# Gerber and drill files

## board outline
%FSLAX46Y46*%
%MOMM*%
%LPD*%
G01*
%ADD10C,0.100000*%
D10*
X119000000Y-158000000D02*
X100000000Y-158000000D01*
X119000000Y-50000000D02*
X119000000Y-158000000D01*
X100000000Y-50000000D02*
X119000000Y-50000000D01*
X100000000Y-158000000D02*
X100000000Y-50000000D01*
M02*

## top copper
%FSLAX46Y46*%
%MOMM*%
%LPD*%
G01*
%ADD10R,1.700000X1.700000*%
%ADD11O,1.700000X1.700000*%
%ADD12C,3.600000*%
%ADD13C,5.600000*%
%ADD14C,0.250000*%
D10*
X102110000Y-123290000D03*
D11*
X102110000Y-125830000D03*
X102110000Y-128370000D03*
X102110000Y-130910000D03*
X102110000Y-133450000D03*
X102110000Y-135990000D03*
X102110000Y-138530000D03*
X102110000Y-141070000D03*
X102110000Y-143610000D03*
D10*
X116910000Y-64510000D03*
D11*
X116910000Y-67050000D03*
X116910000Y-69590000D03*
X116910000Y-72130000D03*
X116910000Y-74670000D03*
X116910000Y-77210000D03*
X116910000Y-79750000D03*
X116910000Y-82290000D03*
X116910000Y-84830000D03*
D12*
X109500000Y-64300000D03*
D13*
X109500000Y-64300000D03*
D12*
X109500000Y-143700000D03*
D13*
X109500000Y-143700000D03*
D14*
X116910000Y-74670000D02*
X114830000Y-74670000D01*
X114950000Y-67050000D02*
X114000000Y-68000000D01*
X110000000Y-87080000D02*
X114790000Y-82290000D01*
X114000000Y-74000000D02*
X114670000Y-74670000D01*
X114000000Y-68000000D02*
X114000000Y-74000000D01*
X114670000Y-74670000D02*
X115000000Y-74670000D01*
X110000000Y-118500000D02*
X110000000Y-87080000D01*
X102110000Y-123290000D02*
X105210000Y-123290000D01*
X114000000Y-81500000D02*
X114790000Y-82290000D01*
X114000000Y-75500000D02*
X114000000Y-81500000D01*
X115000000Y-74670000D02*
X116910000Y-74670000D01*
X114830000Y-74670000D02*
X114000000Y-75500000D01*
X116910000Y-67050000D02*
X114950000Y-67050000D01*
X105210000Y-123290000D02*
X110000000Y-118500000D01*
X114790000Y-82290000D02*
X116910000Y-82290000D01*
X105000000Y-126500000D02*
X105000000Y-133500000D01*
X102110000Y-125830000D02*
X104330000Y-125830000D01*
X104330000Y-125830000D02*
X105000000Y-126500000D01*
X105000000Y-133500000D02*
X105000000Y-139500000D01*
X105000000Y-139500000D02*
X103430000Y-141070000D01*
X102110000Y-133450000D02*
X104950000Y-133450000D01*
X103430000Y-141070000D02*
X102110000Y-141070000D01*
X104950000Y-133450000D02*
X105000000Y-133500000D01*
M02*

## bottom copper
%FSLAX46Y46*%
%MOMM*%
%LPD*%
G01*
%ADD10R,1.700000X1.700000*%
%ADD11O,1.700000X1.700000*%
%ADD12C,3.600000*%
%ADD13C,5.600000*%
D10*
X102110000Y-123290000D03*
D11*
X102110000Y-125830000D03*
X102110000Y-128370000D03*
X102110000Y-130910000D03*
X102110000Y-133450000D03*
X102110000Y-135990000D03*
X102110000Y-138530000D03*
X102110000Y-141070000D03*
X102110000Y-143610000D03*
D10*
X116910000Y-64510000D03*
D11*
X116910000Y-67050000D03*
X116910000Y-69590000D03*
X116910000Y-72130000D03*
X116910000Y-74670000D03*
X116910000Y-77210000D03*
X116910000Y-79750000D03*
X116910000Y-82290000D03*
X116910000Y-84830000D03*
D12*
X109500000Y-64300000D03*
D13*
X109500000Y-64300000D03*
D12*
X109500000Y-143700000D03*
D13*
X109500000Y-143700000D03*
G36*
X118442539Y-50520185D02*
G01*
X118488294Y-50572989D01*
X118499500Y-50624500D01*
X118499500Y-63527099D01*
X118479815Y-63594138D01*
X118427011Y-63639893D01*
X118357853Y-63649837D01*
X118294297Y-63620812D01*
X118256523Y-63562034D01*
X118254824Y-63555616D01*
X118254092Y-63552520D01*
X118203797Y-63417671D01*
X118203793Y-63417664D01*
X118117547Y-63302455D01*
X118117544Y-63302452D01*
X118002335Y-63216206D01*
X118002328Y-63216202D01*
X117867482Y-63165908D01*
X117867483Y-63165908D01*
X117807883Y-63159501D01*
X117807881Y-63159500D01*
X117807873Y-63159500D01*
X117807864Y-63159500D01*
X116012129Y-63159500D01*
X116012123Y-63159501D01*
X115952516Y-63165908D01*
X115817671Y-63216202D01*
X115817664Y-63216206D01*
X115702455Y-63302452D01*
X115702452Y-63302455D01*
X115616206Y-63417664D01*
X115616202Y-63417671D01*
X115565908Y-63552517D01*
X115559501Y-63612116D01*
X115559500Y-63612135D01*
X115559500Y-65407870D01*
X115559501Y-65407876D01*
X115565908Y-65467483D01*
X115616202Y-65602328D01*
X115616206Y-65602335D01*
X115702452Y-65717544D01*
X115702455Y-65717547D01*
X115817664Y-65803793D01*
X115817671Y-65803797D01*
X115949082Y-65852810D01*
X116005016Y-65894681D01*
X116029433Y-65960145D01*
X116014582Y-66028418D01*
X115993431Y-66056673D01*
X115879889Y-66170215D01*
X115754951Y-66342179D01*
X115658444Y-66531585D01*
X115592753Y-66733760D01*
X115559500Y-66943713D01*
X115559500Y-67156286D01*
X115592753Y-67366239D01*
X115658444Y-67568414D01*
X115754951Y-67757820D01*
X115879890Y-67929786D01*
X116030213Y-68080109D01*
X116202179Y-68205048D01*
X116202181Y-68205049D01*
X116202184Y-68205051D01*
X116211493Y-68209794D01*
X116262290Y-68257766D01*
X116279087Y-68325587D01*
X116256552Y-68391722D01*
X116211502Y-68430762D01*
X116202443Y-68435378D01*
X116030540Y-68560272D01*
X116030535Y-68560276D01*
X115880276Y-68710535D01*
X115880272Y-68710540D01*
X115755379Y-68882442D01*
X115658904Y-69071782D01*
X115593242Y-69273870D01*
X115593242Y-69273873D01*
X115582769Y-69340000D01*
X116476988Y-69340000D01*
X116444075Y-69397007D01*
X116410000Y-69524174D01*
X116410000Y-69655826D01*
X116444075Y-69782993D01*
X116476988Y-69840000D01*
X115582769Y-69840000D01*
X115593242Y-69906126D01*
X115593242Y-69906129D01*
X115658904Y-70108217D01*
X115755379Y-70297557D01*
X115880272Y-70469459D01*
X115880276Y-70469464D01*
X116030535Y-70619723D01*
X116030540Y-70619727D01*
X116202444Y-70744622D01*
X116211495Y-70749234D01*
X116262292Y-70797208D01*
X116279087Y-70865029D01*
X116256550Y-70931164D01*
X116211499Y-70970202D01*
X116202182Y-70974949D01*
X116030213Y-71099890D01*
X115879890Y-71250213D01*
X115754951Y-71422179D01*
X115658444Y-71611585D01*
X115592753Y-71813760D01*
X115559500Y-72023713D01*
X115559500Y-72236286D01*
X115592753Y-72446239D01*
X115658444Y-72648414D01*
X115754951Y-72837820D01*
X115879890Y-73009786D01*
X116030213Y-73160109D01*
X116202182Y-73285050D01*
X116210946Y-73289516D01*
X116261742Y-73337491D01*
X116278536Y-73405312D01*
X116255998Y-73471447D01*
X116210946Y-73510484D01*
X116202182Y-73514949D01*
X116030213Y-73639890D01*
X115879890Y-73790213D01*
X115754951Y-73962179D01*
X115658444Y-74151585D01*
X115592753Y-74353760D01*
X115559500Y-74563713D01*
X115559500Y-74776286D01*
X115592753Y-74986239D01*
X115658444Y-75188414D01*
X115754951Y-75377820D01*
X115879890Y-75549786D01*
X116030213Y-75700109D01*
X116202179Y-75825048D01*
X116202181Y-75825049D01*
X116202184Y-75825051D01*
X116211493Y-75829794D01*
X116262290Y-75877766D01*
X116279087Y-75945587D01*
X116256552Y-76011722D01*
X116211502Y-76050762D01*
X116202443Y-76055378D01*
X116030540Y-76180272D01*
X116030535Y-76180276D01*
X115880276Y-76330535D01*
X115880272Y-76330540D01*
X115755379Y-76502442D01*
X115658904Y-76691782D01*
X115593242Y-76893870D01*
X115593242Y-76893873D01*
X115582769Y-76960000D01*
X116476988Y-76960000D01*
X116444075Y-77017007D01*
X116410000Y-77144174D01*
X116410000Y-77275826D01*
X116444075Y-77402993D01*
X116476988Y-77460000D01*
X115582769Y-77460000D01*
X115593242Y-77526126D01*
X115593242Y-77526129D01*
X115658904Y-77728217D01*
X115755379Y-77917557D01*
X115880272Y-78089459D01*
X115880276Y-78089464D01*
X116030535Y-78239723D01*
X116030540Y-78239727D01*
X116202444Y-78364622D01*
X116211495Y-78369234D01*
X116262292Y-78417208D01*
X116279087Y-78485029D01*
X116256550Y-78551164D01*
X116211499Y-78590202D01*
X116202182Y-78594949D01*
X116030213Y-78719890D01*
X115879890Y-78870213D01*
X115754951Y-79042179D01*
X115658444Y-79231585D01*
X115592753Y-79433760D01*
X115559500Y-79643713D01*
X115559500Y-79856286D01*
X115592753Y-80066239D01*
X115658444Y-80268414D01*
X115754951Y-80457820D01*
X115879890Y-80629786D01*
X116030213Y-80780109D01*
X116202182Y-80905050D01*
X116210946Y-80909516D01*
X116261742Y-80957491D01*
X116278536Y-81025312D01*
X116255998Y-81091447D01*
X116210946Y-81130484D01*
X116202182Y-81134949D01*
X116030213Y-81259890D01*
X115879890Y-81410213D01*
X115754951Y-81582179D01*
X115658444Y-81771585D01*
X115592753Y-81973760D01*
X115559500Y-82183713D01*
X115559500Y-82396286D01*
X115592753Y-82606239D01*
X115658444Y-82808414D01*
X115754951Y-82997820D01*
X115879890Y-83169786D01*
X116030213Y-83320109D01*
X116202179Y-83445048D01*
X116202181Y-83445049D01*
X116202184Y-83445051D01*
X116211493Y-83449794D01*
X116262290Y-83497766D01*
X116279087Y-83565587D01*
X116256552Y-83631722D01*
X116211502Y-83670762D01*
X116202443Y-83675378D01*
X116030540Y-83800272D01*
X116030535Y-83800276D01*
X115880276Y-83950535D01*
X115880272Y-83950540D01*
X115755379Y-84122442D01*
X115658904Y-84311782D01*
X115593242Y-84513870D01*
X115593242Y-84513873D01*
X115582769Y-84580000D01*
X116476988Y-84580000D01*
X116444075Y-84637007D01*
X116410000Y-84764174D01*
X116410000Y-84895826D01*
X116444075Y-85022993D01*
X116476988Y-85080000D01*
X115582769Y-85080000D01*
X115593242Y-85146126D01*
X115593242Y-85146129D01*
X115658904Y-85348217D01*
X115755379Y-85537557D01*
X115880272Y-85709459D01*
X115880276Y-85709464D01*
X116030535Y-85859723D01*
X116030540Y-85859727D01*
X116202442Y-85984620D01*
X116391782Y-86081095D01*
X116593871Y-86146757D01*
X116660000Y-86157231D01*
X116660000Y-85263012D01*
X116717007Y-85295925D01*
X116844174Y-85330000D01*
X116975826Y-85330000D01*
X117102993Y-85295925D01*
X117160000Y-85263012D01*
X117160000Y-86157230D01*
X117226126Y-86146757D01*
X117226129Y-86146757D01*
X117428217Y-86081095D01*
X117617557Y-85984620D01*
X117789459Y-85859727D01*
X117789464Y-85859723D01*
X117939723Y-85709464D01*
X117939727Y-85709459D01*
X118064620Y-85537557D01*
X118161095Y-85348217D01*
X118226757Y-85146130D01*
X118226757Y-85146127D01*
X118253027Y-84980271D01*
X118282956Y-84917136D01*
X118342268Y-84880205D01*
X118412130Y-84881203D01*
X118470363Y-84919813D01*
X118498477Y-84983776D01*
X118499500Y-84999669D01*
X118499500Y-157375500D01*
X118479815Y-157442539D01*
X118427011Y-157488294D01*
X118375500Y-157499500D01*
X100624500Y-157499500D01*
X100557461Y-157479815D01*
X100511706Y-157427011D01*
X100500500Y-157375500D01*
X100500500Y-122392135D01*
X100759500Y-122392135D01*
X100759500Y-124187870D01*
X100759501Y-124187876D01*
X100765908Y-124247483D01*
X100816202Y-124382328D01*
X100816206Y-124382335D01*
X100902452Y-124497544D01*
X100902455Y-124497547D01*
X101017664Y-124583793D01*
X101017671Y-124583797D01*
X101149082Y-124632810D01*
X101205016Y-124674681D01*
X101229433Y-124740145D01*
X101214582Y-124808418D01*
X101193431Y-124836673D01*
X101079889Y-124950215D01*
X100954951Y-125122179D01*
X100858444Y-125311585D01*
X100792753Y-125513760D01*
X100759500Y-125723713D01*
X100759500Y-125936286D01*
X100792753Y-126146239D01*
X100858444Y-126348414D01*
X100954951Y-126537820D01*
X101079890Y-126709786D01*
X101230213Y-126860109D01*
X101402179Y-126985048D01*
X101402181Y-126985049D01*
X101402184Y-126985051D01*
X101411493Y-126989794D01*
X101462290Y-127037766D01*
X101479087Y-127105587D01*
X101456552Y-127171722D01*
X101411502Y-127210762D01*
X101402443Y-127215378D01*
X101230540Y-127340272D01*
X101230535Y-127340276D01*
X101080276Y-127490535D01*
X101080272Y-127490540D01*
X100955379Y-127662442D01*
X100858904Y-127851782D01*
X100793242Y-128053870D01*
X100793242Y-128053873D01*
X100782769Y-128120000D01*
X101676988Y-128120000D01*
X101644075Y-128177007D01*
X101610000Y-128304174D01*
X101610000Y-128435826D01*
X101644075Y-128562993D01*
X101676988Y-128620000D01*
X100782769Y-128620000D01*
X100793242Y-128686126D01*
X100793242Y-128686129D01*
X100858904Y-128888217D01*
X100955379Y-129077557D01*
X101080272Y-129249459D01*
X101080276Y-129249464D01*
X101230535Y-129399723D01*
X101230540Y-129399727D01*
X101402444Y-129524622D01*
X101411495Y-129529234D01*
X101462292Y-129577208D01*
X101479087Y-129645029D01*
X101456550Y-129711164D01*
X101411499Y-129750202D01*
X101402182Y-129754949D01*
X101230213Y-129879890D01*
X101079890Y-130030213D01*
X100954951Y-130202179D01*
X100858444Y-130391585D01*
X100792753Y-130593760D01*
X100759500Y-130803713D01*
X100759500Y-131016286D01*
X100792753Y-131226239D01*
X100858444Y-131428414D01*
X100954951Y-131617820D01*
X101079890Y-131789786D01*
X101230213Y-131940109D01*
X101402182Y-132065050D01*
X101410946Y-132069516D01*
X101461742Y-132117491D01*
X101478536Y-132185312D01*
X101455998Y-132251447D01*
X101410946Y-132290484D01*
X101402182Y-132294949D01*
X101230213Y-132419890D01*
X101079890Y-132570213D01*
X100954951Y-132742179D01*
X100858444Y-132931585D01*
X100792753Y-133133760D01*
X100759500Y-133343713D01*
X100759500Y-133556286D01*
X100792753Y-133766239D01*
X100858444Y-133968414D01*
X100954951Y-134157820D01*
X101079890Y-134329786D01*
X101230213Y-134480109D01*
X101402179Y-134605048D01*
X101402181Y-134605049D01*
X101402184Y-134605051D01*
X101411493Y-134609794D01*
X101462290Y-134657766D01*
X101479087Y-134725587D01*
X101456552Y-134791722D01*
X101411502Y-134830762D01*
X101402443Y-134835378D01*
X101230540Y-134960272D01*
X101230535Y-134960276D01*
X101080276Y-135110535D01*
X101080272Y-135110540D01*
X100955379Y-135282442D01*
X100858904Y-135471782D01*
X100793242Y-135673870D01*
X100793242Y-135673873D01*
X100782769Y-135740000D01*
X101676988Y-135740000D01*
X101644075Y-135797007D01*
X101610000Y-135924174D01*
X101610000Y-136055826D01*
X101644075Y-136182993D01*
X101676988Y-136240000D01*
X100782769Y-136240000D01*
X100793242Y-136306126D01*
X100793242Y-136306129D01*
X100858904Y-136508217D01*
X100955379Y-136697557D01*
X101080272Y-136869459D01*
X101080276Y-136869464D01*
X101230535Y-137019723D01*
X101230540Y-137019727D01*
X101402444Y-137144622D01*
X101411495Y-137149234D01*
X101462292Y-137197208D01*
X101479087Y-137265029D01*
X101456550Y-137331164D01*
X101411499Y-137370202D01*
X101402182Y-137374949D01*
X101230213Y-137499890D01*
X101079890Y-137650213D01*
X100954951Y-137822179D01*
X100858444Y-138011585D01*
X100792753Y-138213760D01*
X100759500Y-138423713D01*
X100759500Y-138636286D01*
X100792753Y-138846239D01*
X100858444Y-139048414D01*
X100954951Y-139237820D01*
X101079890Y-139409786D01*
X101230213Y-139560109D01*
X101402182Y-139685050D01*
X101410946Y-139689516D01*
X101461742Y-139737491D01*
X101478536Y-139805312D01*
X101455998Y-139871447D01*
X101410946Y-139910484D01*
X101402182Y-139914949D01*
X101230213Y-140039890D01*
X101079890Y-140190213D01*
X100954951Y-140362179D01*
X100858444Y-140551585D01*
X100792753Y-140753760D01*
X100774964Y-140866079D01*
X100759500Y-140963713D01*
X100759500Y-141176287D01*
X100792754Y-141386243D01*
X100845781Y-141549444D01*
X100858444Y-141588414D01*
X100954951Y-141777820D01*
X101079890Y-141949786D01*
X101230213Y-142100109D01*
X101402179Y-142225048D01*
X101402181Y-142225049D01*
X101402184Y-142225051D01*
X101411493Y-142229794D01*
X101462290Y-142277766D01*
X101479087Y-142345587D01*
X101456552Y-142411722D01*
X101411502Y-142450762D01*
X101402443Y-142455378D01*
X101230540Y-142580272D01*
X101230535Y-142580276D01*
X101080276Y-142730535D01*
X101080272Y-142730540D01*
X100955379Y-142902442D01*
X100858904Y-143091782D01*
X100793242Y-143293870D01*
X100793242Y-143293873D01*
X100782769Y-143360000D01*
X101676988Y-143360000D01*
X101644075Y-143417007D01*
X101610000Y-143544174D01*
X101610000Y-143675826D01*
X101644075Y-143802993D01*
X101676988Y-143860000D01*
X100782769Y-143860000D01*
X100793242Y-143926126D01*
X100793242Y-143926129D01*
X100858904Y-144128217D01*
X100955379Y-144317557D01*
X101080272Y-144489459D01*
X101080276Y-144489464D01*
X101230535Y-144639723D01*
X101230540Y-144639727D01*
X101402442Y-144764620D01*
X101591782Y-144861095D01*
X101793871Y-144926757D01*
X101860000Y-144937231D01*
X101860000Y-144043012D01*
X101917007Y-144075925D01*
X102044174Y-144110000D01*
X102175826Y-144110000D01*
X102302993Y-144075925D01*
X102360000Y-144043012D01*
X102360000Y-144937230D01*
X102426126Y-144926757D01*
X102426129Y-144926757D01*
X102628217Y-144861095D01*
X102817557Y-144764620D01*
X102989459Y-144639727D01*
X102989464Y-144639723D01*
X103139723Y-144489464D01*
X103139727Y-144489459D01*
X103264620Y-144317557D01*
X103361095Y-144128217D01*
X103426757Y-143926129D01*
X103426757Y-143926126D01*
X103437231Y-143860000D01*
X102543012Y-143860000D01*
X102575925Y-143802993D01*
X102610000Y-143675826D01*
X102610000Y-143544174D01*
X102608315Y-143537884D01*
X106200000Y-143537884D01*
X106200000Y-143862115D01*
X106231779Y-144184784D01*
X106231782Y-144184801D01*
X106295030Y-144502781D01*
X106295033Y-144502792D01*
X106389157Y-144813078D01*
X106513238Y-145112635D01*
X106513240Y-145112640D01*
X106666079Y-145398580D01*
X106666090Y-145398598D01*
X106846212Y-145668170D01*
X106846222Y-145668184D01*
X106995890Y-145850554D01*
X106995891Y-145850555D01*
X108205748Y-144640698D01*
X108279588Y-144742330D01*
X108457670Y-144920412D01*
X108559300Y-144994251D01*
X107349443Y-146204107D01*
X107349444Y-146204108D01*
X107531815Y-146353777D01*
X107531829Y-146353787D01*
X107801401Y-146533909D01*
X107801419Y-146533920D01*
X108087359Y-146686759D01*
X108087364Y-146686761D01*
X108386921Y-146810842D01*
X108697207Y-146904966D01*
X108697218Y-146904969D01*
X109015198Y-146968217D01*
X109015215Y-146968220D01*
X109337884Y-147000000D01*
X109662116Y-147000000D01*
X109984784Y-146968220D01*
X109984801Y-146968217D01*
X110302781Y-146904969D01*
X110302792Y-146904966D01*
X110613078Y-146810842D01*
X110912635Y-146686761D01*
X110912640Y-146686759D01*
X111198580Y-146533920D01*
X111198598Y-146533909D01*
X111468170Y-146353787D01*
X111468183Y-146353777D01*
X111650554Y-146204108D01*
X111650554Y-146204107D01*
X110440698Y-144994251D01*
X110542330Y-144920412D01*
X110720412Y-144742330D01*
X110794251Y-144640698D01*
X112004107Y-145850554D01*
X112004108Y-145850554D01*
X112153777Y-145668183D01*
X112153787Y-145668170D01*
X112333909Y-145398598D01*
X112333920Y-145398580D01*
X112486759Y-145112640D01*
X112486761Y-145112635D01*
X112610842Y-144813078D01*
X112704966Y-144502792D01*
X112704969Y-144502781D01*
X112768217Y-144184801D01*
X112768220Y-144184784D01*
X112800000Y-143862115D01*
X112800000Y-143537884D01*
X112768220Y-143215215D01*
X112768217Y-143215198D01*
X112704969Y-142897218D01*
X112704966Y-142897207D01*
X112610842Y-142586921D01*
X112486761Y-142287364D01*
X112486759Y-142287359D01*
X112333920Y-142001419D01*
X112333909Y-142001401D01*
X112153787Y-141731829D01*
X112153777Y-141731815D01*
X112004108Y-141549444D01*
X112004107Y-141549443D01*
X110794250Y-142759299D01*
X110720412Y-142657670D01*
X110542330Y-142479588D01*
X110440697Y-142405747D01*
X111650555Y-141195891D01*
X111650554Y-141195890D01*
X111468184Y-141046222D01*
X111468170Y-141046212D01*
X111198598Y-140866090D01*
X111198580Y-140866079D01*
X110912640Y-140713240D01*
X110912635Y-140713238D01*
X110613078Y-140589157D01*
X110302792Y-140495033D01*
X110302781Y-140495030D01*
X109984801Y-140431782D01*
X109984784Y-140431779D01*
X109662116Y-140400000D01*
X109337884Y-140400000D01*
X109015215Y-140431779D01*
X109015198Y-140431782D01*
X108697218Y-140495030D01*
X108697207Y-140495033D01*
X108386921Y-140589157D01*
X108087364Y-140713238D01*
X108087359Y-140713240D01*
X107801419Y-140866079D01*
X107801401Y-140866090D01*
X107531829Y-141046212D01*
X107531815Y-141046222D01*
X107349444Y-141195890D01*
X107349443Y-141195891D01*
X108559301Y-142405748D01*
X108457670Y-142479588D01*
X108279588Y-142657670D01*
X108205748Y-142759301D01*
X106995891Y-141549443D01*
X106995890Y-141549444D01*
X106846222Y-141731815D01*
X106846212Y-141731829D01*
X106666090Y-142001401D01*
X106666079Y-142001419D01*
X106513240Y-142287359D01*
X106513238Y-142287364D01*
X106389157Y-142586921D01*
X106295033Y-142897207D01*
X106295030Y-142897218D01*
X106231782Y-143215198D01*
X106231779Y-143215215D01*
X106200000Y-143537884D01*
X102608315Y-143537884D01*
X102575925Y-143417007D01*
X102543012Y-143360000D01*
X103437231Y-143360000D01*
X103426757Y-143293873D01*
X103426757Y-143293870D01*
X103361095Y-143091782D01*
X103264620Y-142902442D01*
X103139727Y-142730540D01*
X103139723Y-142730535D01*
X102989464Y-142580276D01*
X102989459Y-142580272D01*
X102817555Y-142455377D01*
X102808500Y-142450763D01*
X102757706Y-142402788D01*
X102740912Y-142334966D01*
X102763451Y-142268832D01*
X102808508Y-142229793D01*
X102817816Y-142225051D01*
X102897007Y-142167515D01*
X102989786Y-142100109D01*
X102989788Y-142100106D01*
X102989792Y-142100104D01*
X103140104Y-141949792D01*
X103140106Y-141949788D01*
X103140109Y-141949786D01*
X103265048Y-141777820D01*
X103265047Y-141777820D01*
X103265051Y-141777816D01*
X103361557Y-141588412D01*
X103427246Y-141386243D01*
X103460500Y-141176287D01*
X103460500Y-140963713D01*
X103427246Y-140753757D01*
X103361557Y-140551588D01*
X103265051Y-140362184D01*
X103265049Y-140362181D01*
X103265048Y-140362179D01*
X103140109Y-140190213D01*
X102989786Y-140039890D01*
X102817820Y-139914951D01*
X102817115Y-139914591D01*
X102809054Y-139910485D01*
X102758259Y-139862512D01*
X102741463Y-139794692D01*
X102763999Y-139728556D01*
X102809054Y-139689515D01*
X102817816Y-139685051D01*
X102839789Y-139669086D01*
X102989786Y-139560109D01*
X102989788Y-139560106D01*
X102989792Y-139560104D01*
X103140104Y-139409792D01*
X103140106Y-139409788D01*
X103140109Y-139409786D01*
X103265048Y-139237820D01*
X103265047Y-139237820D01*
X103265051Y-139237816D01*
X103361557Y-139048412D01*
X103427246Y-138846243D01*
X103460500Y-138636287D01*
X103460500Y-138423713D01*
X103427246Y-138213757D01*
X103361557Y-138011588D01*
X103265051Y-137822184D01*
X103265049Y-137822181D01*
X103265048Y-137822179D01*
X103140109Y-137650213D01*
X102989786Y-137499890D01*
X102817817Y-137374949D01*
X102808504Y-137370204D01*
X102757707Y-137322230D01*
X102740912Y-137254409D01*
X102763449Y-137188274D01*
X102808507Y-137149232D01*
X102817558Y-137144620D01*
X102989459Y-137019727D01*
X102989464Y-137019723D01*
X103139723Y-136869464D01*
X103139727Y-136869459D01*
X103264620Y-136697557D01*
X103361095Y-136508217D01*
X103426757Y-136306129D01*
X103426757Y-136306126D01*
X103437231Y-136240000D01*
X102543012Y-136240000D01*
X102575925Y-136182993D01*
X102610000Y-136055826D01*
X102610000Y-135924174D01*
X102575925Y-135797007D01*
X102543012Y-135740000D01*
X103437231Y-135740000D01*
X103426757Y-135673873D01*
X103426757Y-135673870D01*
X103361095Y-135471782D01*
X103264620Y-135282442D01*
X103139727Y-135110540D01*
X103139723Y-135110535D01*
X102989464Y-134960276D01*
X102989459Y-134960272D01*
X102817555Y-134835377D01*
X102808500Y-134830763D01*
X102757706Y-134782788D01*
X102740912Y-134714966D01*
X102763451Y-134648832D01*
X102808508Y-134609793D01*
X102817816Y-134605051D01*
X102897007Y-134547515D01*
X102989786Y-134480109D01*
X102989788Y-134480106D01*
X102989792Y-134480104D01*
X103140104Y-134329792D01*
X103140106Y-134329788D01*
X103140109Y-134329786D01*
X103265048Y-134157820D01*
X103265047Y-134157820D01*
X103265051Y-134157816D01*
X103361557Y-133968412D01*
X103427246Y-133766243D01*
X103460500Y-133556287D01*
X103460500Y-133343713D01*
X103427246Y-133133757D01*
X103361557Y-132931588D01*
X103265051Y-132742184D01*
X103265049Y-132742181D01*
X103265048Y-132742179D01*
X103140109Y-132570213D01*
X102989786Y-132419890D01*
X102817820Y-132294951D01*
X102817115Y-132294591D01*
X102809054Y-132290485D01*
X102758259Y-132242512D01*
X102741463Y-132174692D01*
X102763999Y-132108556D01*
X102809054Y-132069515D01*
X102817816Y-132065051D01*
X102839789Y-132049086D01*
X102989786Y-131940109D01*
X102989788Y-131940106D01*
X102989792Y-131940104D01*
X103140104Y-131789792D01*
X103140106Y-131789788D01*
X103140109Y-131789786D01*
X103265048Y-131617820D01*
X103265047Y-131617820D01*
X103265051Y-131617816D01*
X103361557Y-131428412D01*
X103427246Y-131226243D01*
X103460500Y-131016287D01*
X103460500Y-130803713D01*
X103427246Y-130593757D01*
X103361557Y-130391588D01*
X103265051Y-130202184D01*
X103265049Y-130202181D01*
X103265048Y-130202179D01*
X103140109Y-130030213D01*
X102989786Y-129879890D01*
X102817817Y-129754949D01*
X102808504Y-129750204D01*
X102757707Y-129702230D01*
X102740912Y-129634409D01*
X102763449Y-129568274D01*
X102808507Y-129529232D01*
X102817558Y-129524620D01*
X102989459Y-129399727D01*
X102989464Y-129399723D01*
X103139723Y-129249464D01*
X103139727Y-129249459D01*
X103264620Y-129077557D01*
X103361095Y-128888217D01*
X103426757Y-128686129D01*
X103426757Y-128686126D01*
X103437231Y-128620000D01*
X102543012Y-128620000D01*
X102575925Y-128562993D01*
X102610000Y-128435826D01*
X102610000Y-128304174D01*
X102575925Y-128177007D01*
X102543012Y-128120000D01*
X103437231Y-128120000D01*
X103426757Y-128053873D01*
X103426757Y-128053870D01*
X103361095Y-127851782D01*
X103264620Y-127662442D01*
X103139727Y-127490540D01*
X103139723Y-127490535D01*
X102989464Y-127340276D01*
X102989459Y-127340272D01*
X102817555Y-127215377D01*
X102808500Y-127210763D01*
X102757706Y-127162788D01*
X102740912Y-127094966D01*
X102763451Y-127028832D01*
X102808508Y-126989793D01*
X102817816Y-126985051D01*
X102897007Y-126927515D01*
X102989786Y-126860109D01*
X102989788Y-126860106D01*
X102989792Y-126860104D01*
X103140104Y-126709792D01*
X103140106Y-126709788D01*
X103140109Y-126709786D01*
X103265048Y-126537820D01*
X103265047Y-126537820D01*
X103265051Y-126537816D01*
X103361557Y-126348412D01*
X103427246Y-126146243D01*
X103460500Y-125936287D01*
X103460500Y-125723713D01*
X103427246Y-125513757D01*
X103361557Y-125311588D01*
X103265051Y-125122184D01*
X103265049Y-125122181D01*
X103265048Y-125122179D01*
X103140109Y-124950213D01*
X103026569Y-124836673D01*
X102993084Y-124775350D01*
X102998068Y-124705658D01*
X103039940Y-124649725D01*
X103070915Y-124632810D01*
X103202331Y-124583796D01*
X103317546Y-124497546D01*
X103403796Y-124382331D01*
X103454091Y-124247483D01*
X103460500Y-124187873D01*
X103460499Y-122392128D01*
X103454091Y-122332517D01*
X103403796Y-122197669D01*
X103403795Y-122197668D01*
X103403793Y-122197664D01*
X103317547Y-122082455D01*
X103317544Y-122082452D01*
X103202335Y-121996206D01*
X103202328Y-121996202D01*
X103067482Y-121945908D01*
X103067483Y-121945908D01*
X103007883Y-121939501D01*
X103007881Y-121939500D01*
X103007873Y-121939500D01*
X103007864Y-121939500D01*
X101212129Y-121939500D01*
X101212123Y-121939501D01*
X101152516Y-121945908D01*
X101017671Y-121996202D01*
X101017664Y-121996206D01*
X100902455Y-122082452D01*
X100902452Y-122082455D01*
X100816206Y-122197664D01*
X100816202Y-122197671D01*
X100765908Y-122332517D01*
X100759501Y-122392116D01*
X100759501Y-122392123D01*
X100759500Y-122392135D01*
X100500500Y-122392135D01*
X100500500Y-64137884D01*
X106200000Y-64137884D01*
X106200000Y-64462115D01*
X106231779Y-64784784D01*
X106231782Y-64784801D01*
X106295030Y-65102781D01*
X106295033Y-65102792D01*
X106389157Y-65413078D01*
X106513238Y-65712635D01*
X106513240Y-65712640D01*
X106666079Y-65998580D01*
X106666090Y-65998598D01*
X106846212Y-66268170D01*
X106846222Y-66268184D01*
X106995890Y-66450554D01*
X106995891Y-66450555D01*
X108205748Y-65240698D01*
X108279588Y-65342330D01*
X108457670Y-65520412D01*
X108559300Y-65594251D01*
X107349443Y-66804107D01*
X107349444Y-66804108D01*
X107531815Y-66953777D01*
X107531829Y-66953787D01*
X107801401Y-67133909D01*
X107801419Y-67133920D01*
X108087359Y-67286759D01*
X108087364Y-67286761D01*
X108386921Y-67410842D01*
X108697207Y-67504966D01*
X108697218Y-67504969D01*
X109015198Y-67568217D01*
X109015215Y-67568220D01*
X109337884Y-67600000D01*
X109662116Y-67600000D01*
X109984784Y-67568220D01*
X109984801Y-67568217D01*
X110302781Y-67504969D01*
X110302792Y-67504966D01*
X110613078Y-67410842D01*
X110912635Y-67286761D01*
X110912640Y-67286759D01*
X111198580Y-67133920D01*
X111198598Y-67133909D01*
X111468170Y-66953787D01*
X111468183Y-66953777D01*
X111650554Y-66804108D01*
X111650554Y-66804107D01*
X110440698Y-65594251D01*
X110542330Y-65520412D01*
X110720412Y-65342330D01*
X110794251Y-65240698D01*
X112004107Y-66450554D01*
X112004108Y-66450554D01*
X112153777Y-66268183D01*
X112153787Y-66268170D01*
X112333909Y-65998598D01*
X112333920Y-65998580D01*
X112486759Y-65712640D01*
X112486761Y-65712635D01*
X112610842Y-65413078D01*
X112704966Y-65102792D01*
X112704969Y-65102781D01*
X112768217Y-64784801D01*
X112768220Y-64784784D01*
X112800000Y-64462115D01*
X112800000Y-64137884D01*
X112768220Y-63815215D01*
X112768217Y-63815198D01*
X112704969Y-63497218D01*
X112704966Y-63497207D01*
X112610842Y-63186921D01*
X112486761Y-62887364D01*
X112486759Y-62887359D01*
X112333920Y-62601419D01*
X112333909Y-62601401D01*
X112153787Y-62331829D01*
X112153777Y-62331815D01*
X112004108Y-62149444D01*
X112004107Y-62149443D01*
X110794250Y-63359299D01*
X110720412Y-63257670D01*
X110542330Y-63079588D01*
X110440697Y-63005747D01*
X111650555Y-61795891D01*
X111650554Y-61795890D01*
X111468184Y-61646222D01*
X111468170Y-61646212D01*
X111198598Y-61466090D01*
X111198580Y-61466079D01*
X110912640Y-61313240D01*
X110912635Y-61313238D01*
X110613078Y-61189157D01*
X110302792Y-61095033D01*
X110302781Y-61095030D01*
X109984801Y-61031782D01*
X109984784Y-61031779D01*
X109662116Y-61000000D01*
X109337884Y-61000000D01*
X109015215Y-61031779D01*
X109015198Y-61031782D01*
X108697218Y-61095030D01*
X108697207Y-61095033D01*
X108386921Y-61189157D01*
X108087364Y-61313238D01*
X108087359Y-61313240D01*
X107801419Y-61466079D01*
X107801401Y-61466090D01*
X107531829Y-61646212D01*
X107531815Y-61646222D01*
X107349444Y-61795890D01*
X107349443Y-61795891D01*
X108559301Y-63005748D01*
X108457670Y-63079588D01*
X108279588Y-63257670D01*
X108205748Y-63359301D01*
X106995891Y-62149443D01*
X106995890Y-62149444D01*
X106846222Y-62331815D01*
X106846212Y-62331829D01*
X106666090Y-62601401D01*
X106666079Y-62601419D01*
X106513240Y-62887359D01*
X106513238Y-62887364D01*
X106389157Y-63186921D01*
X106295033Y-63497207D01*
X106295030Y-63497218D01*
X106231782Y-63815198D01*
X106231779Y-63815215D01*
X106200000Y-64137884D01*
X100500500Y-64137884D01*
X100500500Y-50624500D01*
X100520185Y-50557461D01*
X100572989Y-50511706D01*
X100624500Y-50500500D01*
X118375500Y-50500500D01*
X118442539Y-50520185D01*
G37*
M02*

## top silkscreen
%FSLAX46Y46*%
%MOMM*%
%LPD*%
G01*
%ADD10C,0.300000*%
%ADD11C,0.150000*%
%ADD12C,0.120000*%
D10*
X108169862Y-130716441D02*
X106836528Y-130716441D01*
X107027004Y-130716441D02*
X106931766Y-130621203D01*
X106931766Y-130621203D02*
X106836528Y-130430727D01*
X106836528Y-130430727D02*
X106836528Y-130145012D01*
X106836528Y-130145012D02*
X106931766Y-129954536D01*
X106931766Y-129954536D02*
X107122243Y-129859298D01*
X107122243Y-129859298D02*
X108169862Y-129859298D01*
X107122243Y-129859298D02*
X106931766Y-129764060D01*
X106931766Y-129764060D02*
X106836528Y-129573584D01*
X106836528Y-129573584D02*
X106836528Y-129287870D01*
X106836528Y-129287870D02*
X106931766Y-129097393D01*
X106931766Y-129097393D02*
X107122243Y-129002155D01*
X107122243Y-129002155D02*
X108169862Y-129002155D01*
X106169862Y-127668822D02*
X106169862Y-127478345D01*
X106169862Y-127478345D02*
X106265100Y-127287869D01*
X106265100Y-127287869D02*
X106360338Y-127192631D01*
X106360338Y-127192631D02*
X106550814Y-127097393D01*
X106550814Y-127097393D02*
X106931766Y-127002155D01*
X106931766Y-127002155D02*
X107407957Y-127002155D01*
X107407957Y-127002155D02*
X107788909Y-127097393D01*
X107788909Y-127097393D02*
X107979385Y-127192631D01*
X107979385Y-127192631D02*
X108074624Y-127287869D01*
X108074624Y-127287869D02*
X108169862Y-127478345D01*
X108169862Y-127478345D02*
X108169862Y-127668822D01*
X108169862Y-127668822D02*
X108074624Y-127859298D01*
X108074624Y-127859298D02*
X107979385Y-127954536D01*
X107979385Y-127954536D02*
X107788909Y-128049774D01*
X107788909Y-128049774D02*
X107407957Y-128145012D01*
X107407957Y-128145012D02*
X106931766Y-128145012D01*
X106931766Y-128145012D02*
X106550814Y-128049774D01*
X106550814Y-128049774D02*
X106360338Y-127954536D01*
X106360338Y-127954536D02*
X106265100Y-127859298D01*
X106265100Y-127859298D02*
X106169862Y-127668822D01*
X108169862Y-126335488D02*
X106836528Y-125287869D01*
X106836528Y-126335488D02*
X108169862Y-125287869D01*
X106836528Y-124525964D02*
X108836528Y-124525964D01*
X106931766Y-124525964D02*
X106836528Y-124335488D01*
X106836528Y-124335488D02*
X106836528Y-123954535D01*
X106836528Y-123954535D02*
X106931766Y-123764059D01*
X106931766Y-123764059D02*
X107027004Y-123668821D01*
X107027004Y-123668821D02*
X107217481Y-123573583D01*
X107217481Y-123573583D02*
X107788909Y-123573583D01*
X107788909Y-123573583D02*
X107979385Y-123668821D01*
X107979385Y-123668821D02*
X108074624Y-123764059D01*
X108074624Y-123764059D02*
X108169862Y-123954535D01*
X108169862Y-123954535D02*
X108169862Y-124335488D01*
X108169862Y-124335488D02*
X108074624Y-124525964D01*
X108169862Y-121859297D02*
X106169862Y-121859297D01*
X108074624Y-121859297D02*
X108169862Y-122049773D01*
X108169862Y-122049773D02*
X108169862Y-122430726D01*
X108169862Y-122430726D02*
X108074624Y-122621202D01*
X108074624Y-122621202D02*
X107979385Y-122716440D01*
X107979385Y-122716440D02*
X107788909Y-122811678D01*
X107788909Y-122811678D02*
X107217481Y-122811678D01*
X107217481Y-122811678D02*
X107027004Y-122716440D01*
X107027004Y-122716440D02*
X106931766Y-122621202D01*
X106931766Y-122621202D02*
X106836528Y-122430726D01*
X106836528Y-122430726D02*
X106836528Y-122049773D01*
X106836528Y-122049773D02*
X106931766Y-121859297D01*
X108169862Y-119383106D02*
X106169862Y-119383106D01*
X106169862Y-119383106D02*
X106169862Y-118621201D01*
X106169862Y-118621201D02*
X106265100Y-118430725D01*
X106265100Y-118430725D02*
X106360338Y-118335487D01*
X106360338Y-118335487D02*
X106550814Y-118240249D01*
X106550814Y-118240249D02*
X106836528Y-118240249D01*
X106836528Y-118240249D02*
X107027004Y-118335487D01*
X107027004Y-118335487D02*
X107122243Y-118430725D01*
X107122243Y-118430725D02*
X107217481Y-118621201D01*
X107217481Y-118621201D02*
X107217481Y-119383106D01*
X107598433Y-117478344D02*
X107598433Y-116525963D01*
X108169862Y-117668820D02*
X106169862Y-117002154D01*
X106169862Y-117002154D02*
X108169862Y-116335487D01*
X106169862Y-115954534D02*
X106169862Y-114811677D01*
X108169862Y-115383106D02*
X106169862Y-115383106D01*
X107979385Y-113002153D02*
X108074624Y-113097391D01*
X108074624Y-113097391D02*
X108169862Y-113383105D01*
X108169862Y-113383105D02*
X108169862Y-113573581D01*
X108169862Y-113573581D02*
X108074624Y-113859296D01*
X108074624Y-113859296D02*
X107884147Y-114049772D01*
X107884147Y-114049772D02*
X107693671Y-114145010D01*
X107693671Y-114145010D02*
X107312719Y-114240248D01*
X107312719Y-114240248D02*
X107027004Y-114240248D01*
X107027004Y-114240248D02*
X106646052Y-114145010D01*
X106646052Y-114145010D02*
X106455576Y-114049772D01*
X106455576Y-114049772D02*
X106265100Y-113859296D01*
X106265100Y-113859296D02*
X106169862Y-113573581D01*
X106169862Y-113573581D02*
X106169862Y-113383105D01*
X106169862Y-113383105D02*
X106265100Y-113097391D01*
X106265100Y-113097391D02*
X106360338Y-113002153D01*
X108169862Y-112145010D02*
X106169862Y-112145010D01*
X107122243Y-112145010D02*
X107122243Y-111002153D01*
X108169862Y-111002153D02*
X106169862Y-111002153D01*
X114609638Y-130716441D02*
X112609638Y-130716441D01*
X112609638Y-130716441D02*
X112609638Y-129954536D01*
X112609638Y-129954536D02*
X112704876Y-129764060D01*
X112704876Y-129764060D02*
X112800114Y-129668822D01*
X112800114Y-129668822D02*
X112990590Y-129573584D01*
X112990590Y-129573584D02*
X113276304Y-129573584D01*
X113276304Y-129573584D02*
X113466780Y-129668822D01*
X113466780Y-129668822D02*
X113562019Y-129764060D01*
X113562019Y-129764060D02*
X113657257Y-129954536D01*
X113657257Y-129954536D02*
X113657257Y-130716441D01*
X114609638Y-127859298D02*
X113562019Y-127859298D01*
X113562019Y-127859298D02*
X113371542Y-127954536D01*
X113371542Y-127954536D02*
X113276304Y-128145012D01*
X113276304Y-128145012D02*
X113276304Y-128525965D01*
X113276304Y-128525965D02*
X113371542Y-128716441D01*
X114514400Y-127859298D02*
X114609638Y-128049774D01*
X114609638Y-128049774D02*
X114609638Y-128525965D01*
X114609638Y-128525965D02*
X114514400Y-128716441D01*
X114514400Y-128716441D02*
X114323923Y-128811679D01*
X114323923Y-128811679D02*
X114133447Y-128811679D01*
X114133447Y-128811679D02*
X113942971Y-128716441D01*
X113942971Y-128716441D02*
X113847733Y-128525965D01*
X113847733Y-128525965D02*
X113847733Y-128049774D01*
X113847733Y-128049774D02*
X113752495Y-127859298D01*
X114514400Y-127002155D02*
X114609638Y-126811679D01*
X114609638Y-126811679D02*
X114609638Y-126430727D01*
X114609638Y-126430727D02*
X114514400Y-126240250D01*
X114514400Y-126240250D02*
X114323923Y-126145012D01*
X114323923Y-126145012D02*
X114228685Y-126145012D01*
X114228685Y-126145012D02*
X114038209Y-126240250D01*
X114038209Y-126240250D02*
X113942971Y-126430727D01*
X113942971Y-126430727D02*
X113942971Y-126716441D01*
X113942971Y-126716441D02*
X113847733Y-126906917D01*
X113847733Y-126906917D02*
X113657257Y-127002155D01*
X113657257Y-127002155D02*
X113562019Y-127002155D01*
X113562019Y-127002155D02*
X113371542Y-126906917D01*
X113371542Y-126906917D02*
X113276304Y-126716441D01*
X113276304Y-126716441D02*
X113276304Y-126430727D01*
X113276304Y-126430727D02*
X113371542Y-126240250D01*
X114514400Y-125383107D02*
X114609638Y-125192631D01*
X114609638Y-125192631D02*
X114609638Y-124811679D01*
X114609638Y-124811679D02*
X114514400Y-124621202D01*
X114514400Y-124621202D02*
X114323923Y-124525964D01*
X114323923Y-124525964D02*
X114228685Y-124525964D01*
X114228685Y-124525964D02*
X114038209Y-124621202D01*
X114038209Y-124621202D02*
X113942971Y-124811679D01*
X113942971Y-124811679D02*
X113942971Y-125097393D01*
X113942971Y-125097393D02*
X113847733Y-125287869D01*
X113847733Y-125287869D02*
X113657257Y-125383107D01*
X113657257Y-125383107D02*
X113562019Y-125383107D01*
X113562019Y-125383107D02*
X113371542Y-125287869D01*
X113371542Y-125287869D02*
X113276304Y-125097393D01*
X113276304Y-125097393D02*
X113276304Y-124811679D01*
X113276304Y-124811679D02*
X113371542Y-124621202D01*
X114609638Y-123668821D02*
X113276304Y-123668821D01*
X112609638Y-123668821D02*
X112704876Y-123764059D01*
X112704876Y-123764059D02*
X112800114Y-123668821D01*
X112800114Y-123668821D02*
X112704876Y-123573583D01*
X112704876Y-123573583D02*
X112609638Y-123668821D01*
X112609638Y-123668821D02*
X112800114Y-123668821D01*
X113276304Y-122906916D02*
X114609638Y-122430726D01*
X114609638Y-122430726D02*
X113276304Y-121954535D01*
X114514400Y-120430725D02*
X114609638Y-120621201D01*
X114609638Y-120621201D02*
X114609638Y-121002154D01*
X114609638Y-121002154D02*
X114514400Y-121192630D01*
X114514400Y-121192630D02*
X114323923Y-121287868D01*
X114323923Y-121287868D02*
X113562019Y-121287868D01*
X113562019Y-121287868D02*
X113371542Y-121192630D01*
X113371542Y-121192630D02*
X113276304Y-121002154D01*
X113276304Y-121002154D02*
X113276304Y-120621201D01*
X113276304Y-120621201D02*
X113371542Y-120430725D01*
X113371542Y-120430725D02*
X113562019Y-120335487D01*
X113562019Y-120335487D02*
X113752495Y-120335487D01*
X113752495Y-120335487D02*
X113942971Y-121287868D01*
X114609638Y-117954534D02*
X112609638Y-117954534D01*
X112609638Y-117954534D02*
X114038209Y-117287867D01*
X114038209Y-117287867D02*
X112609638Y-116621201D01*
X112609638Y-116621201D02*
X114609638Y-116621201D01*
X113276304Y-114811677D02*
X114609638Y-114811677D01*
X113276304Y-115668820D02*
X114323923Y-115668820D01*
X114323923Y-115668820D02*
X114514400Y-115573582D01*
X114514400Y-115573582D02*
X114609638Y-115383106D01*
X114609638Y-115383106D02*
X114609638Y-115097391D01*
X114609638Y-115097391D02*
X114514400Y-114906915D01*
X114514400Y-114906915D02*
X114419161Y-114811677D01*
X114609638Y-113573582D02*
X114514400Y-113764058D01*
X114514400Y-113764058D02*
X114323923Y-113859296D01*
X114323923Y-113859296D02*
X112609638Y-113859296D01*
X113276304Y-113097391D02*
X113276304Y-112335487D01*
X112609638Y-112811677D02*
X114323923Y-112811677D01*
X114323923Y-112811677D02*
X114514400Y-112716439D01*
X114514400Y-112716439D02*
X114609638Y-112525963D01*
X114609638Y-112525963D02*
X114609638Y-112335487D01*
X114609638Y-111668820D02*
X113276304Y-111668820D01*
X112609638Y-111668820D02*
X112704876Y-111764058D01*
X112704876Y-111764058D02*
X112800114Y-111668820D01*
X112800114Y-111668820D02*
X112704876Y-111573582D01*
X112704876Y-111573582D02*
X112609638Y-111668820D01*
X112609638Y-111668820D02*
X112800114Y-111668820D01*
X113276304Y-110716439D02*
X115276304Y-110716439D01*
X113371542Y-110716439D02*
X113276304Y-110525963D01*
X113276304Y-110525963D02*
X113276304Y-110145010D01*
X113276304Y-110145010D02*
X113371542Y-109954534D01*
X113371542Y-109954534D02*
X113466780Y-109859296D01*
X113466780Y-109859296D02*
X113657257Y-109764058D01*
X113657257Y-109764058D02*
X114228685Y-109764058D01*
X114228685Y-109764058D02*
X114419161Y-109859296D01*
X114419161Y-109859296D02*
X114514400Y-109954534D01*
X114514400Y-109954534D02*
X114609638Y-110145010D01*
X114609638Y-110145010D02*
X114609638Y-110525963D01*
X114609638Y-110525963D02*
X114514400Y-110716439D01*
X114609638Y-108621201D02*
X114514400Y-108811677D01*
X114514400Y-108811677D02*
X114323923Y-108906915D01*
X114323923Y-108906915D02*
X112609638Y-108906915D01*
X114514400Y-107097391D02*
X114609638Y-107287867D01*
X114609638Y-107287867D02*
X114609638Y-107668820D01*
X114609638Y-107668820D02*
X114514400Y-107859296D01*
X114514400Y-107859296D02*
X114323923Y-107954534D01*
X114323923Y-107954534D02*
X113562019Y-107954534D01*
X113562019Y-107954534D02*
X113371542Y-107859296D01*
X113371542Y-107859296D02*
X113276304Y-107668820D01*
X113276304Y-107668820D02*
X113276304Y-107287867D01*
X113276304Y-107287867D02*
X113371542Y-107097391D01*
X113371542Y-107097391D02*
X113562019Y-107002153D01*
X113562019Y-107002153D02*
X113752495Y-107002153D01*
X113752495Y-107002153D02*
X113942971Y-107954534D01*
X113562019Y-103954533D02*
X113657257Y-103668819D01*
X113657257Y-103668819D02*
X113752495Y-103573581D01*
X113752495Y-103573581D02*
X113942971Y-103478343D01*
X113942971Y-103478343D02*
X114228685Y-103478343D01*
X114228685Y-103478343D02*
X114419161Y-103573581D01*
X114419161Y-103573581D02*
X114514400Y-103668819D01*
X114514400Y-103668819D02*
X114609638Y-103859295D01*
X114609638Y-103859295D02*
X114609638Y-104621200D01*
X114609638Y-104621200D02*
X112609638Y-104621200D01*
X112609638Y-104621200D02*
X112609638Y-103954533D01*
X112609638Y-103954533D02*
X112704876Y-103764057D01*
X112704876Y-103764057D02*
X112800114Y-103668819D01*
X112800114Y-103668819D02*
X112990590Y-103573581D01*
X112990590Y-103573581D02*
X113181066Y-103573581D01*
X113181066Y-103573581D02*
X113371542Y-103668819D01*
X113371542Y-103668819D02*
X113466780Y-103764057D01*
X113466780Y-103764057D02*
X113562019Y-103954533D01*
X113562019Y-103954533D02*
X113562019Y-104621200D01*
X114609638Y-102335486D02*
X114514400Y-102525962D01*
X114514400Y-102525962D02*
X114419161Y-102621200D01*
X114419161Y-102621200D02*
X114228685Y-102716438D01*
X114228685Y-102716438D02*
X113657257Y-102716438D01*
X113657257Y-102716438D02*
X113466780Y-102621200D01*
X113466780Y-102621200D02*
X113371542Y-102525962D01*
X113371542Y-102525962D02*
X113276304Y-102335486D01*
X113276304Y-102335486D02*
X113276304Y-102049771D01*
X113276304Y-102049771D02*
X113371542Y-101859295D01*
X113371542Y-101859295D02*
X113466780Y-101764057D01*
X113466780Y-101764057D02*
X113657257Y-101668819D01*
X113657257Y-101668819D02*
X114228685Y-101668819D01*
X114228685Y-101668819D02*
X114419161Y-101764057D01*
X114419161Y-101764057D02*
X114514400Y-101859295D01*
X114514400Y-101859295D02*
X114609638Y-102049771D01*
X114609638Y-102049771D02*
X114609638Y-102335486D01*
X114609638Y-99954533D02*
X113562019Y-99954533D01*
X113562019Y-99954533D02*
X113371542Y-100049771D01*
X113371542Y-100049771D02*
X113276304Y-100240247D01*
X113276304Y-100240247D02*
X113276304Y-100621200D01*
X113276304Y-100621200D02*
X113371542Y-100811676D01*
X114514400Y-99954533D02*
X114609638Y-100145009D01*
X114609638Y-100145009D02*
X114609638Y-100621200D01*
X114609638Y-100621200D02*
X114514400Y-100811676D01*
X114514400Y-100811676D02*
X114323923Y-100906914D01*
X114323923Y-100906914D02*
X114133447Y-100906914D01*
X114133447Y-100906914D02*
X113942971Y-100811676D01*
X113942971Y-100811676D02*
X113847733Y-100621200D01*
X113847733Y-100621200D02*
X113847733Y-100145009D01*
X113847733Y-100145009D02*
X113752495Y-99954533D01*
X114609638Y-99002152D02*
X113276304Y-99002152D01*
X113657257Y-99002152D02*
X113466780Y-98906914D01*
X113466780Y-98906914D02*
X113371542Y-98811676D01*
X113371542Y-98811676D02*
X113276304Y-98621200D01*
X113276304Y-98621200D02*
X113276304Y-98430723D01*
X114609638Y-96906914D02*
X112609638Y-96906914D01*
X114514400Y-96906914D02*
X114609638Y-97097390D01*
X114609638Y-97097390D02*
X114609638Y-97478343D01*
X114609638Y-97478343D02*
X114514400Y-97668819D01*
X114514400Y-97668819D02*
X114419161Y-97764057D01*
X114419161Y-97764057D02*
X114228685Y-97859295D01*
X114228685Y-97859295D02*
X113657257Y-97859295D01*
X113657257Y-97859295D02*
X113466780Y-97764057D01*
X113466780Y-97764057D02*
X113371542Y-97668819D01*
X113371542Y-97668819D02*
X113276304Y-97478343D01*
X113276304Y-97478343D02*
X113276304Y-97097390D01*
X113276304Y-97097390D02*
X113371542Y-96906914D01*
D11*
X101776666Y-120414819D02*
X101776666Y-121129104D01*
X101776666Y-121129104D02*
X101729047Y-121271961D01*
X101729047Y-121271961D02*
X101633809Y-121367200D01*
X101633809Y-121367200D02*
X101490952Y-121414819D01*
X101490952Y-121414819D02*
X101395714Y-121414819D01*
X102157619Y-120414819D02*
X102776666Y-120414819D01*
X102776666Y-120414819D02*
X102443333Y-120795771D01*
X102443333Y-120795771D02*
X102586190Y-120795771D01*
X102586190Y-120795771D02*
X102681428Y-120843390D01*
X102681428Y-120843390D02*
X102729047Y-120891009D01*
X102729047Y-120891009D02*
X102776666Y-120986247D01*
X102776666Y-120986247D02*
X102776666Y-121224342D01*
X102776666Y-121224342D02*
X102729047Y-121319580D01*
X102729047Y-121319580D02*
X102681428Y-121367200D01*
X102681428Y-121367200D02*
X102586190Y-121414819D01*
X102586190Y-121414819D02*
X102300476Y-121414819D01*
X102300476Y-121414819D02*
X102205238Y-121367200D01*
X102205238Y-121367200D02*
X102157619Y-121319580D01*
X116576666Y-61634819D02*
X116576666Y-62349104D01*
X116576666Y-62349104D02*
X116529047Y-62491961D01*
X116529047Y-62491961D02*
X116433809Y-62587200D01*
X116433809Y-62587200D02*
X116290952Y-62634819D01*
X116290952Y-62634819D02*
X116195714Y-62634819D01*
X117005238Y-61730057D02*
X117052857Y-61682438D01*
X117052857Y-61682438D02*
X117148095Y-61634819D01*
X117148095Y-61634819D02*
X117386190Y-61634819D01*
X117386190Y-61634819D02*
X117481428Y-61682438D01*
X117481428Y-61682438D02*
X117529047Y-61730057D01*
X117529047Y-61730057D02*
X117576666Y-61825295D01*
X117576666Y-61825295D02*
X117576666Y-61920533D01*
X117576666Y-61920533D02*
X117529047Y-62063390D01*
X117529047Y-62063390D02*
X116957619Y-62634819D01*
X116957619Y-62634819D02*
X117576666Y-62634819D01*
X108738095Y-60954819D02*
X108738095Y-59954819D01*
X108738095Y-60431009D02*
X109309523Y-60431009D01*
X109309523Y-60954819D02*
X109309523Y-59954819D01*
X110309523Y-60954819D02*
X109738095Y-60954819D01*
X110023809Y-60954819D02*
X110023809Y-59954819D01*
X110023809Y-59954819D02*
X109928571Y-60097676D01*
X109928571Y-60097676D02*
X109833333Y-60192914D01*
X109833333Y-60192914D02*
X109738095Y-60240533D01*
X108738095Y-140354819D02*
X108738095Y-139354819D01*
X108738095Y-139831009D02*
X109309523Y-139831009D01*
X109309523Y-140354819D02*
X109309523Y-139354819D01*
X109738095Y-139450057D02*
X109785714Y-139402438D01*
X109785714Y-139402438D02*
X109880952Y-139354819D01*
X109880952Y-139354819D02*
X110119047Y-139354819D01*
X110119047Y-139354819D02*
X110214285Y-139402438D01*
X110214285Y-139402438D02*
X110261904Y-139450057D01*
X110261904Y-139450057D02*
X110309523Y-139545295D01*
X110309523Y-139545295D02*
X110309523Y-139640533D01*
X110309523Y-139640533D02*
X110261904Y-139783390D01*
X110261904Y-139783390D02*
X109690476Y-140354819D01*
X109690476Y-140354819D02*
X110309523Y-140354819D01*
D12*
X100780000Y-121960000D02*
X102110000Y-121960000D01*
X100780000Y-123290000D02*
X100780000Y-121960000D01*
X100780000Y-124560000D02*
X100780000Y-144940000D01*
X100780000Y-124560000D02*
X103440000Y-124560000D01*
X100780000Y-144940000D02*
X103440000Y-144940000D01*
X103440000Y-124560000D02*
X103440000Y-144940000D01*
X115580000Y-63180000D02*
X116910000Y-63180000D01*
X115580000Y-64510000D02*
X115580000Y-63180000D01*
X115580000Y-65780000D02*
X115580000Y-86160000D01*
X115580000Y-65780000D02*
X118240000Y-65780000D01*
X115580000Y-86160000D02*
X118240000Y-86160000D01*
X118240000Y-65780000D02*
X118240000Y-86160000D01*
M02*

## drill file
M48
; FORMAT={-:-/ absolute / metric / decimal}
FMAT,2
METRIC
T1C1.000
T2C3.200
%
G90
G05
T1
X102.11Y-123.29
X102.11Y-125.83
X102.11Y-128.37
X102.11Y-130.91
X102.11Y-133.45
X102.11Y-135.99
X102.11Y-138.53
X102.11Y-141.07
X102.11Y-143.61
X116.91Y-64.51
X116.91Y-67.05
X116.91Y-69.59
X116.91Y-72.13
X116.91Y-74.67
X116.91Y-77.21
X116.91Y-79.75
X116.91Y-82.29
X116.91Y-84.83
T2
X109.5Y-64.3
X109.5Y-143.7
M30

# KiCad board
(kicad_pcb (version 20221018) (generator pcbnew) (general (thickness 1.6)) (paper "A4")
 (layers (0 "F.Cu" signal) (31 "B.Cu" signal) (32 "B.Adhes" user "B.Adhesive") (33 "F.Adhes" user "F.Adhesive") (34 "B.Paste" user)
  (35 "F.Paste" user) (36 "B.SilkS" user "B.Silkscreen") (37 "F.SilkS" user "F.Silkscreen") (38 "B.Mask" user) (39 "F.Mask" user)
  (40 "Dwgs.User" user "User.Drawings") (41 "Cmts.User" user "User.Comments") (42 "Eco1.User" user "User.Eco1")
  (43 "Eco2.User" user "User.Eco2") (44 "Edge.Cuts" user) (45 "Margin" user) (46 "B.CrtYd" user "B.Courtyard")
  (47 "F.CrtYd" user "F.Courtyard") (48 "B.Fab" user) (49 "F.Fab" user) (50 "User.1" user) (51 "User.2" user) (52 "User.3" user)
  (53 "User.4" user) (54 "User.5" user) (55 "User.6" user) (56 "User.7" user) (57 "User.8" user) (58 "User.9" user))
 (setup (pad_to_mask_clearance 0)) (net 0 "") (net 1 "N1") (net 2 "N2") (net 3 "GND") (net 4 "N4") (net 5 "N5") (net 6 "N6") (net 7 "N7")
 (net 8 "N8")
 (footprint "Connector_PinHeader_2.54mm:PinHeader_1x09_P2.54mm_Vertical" (layer "F.Cu") (at 102.11 123.29)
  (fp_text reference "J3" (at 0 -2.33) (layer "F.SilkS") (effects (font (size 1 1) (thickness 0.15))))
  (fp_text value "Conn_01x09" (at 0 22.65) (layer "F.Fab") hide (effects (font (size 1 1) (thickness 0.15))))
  (fp_line (start -1.33 -1.33) (end 0 -1.33) (stroke (width 0.12) (type solid)) (layer "F.SilkS"))
  (fp_line (start -1.33 0) (end -1.33 -1.33) (stroke (width 0.12) (type solid)) (layer "F.SilkS"))
  (fp_line (start -1.33 1.27) (end -1.33 21.65) (stroke (width 0.12) (type solid)) (layer "F.SilkS"))
  (fp_line (start -1.33 1.27) (end 1.33 1.27) (stroke (width 0.12) (type solid)) (layer "F.SilkS"))
  (fp_line (start -1.33 21.65) (end 1.33 21.65) (stroke (width 0.12) (type solid)) (layer "F.SilkS"))
  (fp_line (start 1.33 1.27) (end 1.33 21.65) (stroke (width 0.12) (type solid)) (layer "F.SilkS"))
  (pad "1" thru_hole rect (at 0 0) (size 1.7 1.7) (drill 1) (layers "*.Cu" "*.Mask") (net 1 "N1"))
  (pad "2" thru_hole oval (at 0 2.54) (size 1.7 1.7) (drill 1) (layers "*.Cu" "*.Mask") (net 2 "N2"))
  (pad "3" thru_hole oval (at 0 5.08) (size 1.7 1.7) (drill 1) (layers "*.Cu" "*.Mask") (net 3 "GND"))
  (pad "4" thru_hole oval (at 0 7.62) (size 1.7 1.7) (drill 1) (layers "*.Cu" "*.Mask") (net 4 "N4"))
  (pad "5" thru_hole oval (at 0 10.16) (size 1.7 1.7) (drill 1) (layers "*.Cu" "*.Mask") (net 2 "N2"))
  (pad "6" thru_hole oval (at 0 12.7) (size 1.7 1.7) (drill 1) (layers "*.Cu" "*.Mask") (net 3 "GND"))
  (pad "7" thru_hole oval (at 0 15.24) (size 1.7 1.7) (drill 1) (layers "*.Cu" "*.Mask") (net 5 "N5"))
  (pad "8" thru_hole oval (at 0 17.78) (size 1.7 1.7) (drill 1) (layers "*.Cu" "*.Mask") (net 2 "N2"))
  (pad "9" thru_hole oval (at 0 20.32) (size 1.7 1.7) (drill 1) (layers "*.Cu" "*.Mask") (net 3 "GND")))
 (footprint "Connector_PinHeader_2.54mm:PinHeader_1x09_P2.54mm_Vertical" (layer "F.Cu") (at 116.91 64.51)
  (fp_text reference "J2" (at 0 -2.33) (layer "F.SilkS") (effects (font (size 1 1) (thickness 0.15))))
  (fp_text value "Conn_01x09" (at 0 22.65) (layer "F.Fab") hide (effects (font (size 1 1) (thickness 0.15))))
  (fp_line (start -1.33 -1.33) (end 0 -1.33) (stroke (width 0.12) (type solid)) (layer "F.SilkS"))
  (fp_line (start -1.33 0) (end -1.33 -1.33) (stroke (width 0.12) (type solid)) (layer "F.SilkS"))
  (fp_line (start -1.33 1.27) (end -1.33 21.65) (stroke (width 0.12) (type solid)) (layer "F.SilkS"))
  (fp_line (start -1.33 1.27) (end 1.33 1.27) (stroke (width 0.12) (type solid)) (layer "F.SilkS"))
  (fp_line (start -1.33 21.65) (end 1.33 21.65) (stroke (width 0.12) (type solid)) (layer "F.SilkS"))
  (fp_line (start 1.33 1.27) (end 1.33 21.65) (stroke (width 0.12) (type solid)) (layer "F.SilkS"))
  (pad "1" thru_hole rect (at 0 0) (size 1.7 1.7) (drill 1) (layers "*.Cu" "*.Mask") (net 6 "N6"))
  (pad "2" thru_hole oval (at 0 2.54) (size 1.7 1.7) (drill 1) (layers "*.Cu" "*.Mask") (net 1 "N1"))
  (pad "3" thru_hole oval (at 0 5.08) (size 1.7 1.7) (drill 1) (layers "*.Cu" "*.Mask") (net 3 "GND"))
  (pad "4" thru_hole oval (at 0 7.62) (size 1.7 1.7) (drill 1) (layers "*.Cu" "*.Mask") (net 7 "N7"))
  (pad "5" thru_hole oval (at 0 10.16) (size 1.7 1.7) (drill 1) (layers "*.Cu" "*.Mask") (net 1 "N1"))
  (pad "6" thru_hole oval (at 0 12.7) (size 1.7 1.7) (drill 1) (layers "*.Cu" "*.Mask") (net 3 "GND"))
  (pad "7" thru_hole oval (at 0 15.24) (size 1.7 1.7) (drill 1) (layers "*.Cu" "*.Mask") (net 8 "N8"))
  (pad "8" thru_hole oval (at 0 17.78) (size 1.7 1.7) (drill 1) (layers "*.Cu" "*.Mask") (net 1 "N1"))
  (pad "9" thru_hole oval (at 0 20.32) (size 1.7 1.7) (drill 1) (layers "*.Cu" "*.Mask") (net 3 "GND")))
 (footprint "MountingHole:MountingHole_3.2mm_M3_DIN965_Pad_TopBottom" (layer "F.Cu") (at 109.5 64.3)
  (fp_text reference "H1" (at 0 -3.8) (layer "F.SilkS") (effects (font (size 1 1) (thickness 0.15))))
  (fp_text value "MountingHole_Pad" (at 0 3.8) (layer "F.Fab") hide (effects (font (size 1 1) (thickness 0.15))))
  (pad "1" thru_hole circle (at 0 0) (size 3.6 3.6) (drill 3.2) (layers "*.Cu" "*.Mask") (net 3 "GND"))
  (pad "1" connect circle (at 0 0) (size 5.6 5.6) (layers "F.Cu" "F.Mask") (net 3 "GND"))
  (pad "1" connect circle (at 0 0) (size 5.6 5.6) (layers "B.Cu" "B.Mask") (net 3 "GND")))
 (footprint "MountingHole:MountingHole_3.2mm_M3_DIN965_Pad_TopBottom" (layer "F.Cu") (at 109.5 143.7)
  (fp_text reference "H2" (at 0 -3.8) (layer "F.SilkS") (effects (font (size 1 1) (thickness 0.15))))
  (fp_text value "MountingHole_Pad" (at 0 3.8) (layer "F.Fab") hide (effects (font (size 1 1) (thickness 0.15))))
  (pad "1" thru_hole circle (at 0 0) (size 3.6 3.6) (drill 3.2) (layers "*.Cu" "*.Mask") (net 3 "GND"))
  (pad "1" connect circle (at 0 0) (size 5.6 5.6) (layers "F.Cu" "F.Mask") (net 3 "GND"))
  (pad "1" connect circle (at 0 0) (size 5.6 5.6) (layers "B.Cu" "B.Mask") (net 3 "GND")))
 (gr_line (start 119 158) (end 100 158) (stroke (width 0.1) (type default)) (layer "Edge.Cuts"))
 (gr_line (start 119 50) (end 119 158) (stroke (width 0.1) (type default)) (layer "Edge.Cuts"))
 (gr_line (start 100 50) (end 119 50) (stroke (width 0.1) (type default)) (layer "Edge.Cuts"))
 (gr_line (start 100 158) (end 100 50) (stroke (width 0.1) (type default)) (layer "Edge.Cuts"))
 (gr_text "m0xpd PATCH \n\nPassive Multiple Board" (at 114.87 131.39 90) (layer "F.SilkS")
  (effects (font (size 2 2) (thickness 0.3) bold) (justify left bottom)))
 (segment (start 116.91 74.67) (end 114.83 74.67) (width 0.25) (layer "F.Cu") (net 1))
 (segment (start 114.95 67.05) (end 114 68) (width 0.25) (layer "F.Cu") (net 1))
 (segment (start 110 87.08) (end 114.79 82.29) (width 0.25) (layer "F.Cu") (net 1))
 (segment (start 114 74) (end 114.67 74.67) (width 0.25) (layer "F.Cu") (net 1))
 (segment (start 114 68) (end 114 74) (width 0.25) (layer "F.Cu") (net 1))
 (segment (start 114.67 74.67) (end 115 74.67) (width 0.25) (layer "F.Cu") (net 1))
 (segment (start 110 118.5) (end 110 87.08) (width 0.25) (layer "F.Cu") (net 1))
 (segment (start 102.11 123.29) (end 105.21 123.29) (width 0.25) (layer "F.Cu") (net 1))
 (segment (start 114 81.5) (end 114.79 82.29) (width 0.25) (layer "F.Cu") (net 1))
 (segment (start 114 75.5) (end 114 81.5) (width 0.25) (layer "F.Cu") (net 1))
 (segment (start 115 74.67) (end 116.91 74.67) (width 0.25) (layer "F.Cu") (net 1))
 (segment (start 114.83 74.67) (end 114 75.5) (width 0.25) (layer "F.Cu") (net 1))
 (segment (start 116.91 67.05) (end 114.95 67.05) (width 0.25) (layer "F.Cu") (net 1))
 (segment (start 105.21 123.29) (end 110 118.5) (width 0.25) (layer "F.Cu") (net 1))
 (segment (start 114.79 82.29) (end 116.91 82.29) (width 0.25) (layer "F.Cu") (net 1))
 (segment (start 105 126.5) (end 105 133.5) (width 0.25) (layer "F.Cu") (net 2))
 (segment (start 102.11 125.83) (end 104.33 125.83) (width 0.25) (layer "F.Cu") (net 2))
 (segment (start 104.33 125.83) (end 105 126.5) (width 0.25) (layer "F.Cu") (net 2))
 (segment (start 105 133.5) (end 105 139.5) (width 0.25) (layer "F.Cu") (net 2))
 (segment (start 105 139.5) (end 103.43 141.07) (width 0.25) (layer "F.Cu") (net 2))
 (segment (start 102.11 133.45) (end 104.95 133.45) (width 0.25) (layer "F.Cu") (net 2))
 (segment (start 103.43 141.07) (end 102.11 141.07) (width 0.25) (layer "F.Cu") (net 2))
 (segment (start 104.95 133.45) (end 105 133.5) (width 0.25) (layer "F.Cu") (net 2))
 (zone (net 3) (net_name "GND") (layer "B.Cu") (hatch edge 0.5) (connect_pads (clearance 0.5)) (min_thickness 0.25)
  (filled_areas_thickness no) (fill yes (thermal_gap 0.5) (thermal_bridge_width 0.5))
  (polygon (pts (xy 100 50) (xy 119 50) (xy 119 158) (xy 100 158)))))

